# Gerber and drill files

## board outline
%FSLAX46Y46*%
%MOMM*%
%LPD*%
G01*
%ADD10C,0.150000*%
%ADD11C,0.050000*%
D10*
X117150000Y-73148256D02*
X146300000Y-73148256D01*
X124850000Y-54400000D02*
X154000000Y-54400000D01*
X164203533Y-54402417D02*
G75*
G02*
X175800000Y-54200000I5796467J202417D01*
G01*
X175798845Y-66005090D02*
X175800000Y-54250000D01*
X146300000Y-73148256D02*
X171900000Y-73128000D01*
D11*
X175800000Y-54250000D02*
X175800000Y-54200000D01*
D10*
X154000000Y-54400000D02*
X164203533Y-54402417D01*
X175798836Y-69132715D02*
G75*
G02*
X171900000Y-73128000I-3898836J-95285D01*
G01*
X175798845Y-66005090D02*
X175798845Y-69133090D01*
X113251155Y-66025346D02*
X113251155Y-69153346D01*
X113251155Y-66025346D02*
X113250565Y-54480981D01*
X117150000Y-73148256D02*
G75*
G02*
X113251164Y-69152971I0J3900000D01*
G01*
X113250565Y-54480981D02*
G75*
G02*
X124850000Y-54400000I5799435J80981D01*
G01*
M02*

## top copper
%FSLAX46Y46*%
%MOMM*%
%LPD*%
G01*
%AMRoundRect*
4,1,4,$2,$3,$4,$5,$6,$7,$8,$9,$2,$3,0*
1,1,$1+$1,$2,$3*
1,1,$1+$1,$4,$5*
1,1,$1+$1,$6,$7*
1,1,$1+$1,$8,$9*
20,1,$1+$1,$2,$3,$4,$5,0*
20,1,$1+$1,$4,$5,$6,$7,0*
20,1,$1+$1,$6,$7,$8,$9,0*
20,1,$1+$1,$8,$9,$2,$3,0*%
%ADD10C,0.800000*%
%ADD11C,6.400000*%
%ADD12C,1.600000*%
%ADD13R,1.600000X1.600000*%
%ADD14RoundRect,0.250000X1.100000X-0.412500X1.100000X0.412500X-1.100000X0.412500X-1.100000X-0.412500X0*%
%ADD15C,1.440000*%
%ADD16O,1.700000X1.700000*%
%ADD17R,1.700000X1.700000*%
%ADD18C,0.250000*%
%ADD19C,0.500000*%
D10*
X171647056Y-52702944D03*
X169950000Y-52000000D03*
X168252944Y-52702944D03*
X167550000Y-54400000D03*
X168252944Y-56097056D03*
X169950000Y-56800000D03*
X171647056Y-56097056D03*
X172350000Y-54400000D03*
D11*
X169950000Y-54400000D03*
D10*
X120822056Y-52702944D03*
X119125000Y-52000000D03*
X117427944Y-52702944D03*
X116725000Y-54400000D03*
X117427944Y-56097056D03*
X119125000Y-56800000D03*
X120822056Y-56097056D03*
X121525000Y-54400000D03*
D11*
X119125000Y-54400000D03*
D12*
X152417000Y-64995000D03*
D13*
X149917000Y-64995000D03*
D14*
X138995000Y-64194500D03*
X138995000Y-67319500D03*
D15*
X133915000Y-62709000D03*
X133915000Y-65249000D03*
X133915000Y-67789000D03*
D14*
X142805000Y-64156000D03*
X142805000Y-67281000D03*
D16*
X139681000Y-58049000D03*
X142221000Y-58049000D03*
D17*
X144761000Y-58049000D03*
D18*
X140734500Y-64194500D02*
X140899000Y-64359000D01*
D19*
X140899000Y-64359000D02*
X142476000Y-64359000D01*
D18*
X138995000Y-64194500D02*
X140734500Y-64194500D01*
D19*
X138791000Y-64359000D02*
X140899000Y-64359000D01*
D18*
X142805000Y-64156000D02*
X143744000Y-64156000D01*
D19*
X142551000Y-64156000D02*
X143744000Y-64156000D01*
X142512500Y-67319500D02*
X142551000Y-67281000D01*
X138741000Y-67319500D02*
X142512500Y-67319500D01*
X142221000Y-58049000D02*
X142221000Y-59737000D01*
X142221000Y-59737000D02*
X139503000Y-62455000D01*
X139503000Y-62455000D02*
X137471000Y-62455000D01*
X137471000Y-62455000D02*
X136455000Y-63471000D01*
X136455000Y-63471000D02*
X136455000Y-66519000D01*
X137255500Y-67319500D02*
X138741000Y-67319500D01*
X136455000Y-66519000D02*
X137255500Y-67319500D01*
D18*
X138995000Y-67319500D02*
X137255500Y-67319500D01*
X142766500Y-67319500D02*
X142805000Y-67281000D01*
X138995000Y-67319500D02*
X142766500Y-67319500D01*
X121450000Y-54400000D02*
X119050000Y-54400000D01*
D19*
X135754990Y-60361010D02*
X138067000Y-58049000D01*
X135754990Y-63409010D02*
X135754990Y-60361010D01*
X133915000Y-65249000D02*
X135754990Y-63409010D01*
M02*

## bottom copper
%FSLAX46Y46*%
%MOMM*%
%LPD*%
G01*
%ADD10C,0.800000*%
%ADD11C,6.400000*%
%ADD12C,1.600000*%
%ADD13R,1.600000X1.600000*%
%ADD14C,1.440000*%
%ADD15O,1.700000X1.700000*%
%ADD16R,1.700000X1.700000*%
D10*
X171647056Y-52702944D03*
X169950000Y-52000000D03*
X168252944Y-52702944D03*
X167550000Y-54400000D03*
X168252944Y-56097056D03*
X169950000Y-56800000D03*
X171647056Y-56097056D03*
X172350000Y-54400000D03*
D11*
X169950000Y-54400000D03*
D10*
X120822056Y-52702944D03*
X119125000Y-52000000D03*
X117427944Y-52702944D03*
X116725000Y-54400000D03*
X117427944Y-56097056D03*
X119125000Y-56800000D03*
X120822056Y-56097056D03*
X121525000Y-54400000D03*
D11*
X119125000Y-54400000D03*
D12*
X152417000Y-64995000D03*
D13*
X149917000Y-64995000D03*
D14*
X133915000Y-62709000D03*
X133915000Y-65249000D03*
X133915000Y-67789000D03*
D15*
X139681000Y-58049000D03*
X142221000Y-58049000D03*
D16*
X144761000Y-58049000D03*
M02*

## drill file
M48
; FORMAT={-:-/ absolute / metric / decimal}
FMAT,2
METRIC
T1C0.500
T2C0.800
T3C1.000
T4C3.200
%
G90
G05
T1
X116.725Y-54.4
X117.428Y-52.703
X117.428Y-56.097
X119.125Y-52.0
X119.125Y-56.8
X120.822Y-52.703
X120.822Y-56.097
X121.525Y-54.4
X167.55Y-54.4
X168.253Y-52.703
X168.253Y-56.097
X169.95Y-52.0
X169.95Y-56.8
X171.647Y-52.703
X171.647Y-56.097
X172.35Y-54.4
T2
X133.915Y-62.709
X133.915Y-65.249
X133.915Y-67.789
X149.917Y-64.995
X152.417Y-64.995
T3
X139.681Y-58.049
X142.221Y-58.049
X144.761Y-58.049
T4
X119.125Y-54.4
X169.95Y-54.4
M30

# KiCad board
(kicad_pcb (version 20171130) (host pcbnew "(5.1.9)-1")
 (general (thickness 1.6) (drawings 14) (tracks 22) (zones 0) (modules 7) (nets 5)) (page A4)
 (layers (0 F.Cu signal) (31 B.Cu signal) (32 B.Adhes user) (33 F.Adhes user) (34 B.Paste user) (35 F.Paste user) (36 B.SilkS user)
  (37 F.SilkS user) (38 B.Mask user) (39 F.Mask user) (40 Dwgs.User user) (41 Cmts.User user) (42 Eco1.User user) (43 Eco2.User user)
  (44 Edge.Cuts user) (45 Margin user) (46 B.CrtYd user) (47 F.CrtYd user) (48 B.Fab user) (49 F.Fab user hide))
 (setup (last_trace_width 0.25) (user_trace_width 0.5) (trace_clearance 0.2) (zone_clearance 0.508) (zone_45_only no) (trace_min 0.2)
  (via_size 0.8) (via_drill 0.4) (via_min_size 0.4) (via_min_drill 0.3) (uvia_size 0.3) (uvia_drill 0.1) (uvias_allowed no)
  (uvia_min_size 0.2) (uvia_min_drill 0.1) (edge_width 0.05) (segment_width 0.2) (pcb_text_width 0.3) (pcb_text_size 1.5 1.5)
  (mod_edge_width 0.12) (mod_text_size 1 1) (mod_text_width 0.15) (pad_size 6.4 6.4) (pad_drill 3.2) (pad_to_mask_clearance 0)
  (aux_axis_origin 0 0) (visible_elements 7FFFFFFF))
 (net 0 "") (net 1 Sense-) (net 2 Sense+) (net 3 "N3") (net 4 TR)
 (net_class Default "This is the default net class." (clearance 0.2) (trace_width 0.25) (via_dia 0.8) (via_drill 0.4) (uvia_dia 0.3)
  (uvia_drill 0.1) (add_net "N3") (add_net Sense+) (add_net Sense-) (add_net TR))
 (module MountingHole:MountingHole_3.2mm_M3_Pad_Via (layer F.Cu) (at 169.95 54.4)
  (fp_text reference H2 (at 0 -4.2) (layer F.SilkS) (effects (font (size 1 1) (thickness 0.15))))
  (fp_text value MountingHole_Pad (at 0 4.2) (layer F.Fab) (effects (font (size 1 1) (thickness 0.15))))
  (pad 1 thru_hole circle (at 1.697056 -1.697056) (size 0.8 0.8) (drill 0.5) (layers *.Cu *.Mask) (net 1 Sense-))
  (pad 1 thru_hole circle (at 0 -2.4) (size 0.8 0.8) (drill 0.5) (layers *.Cu *.Mask) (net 1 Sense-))
  (pad 1 thru_hole circle (at -1.697056 -1.697056) (size 0.8 0.8) (drill 0.5) (layers *.Cu *.Mask) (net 1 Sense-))
  (pad 1 thru_hole circle (at -2.4 0) (size 0.8 0.8) (drill 0.5) (layers *.Cu *.Mask) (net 1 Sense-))
  (pad 1 thru_hole circle (at -1.697056 1.697056) (size 0.8 0.8) (drill 0.5) (layers *.Cu *.Mask) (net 1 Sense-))
  (pad 1 thru_hole circle (at 0 2.4) (size 0.8 0.8) (drill 0.5) (layers *.Cu *.Mask) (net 1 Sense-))
  (pad 1 thru_hole circle (at 1.697056 1.697056) (size 0.8 0.8) (drill 0.5) (layers *.Cu *.Mask) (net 1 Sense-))
  (pad 1 thru_hole circle (at 2.4 0) (size 0.8 0.8) (drill 0.5) (layers *.Cu *.Mask) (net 1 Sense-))
  (pad 1 thru_hole circle (at 0 0) (size 6.4 6.4) (drill 3.2) (layers *.Cu *.Mask) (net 1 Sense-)))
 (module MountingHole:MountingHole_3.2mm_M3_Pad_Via (layer F.Cu) (at 119.125 54.4)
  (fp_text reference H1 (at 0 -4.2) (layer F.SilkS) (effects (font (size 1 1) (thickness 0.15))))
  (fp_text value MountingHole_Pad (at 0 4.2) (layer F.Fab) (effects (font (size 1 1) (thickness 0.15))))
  (pad 1 thru_hole circle (at 1.697056 -1.697056) (size 0.8 0.8) (drill 0.5) (layers *.Cu *.Mask) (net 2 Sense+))
  (pad 1 thru_hole circle (at 0 -2.4) (size 0.8 0.8) (drill 0.5) (layers *.Cu *.Mask) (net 2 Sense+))
  (pad 1 thru_hole circle (at -1.697056 -1.697056) (size 0.8 0.8) (drill 0.5) (layers *.Cu *.Mask) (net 2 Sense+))
  (pad 1 thru_hole circle (at -2.4 0) (size 0.8 0.8) (drill 0.5) (layers *.Cu *.Mask) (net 2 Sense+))
  (pad 1 thru_hole circle (at -1.697056 1.697056) (size 0.8 0.8) (drill 0.5) (layers *.Cu *.Mask) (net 2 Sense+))
  (pad 1 thru_hole circle (at 0 2.4) (size 0.8 0.8) (drill 0.5) (layers *.Cu *.Mask) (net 2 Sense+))
  (pad 1 thru_hole circle (at 1.697056 1.697056) (size 0.8 0.8) (drill 0.5) (layers *.Cu *.Mask) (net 2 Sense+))
  (pad 1 thru_hole circle (at 2.4 0) (size 0.8 0.8) (drill 0.5) (layers *.Cu *.Mask) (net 2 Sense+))
  (pad 1 thru_hole circle (at 0 0) (size 6.4 6.4) (drill 3.2) (layers *.Cu *.Mask) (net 2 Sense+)))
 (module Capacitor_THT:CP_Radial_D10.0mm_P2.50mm (layer F.Cu) (at 149.917 64.995)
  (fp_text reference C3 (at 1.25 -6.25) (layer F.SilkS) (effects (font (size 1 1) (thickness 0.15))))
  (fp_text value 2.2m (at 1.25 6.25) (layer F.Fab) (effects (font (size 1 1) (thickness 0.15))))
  (pad 2 thru_hole circle (at 2.5 0) (size 1.6 1.6) (drill 0.8) (layers *.Cu *.Mask) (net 1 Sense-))
  (pad 1 thru_hole rect (at 0 0) (size 1.6 1.6) (drill 0.8) (layers *.Cu *.Mask) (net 2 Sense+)))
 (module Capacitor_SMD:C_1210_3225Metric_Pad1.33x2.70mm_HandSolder (layer F.Cu) (at 138.995 65.757 90)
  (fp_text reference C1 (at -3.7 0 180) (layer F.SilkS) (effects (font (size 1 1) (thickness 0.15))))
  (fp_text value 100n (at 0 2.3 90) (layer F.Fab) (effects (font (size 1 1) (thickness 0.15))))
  (pad 2 smd roundrect (at 1.5625 0 90) (size 1.325 2.7) (layers F.Cu F.Paste F.Mask) (roundrect_rratio 0.188679) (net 1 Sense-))
  (pad 1 smd roundrect (at -1.5625 0 90) (size 1.325 2.7) (layers F.Cu F.Paste F.Mask) (roundrect_rratio 0.188679) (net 2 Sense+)))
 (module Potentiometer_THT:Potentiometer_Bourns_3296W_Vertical (layer F.Cu) (at 133.915 67.789 270)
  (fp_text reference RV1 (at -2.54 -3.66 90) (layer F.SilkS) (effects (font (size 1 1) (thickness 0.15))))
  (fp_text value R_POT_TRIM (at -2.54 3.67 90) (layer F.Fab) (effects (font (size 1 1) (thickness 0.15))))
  (pad 3 thru_hole circle (at -5.08 0 270) (size 1.44 1.44) (drill 0.8) (layers *.Cu *.Mask) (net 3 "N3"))
  (pad 2 thru_hole circle (at -2.54 0 270) (size 1.44 1.44) (drill 0.8) (layers *.Cu *.Mask) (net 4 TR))
  (pad 1 thru_hole circle (at 0 0 270) (size 1.44 1.44) (drill 0.8) (layers *.Cu *.Mask) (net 1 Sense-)))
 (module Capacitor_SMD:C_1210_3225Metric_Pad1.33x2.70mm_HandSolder (layer F.Cu) (at 142.805 65.7185 90)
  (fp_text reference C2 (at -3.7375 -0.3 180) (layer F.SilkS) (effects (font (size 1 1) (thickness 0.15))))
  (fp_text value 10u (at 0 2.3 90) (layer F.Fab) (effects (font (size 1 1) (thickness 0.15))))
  (pad 2 smd roundrect (at 1.5625 0 90) (size 1.325 2.7) (layers F.Cu F.Paste F.Mask) (roundrect_rratio 0.188679) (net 1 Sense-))
  (pad 1 smd roundrect (at -1.5625 0 90) (size 1.325 2.7) (layers F.Cu F.Paste F.Mask) (roundrect_rratio 0.188679) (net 2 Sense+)))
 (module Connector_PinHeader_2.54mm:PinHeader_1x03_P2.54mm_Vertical (layer F.Cu) (at 144.761 58.049 270)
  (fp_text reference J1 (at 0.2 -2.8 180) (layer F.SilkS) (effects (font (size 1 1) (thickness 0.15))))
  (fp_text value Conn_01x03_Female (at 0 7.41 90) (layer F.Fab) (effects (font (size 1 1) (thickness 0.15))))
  (pad 3 thru_hole oval (at 0 5.08 270) (size 1.7 1.7) (drill 1) (layers *.Cu *.Mask) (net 4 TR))
  (pad 2 thru_hole oval (at 0 2.54 270) (size 1.7 1.7) (drill 1) (layers *.Cu *.Mask) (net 2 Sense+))
  (pad 1 thru_hole rect (at 0 0 270) (size 1.7 1.7) (drill 1) (layers *.Cu *.Mask) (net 1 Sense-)))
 (gr_line (start 117.15 73.148256) (end 146.3 73.148256) (layer Edge.Cuts) (width 0.15))
 (gr_line (start 124.85 54.4) (end 154 54.4) (layer Edge.Cuts) (width 0.15))
 (gr_arc (start 170 54.2) (end 175.8 54.2) (angle -182) (layer Edge.Cuts) (width 0.15))
 (gr_line (start 175.798845 66.00509) (end 175.8 54.25) (layer Edge.Cuts) (width 0.15))
 (gr_line (start 146.3 73.148256) (end 171.9 73.128) (layer Edge.Cuts) (width 0.15))
 (gr_line (start 175.8 54.25) (end 175.8 54.2) (layer Edge.Cuts) (width 0.05))
 (gr_line (start 154 54.4) (end 164.203533 54.402417) (layer Edge.Cuts) (width 0.15))
 (gr_arc (start 171.9 69.228) (end 171.9 73.128) (angle -91.4) (layer Edge.Cuts) (width 0.15))
 (gr_line (start 175.798845 66.00509) (end 175.798845 69.13309) (layer Edge.Cuts) (width 0.15))
 (gr_line (start 113.251155 66.025346) (end 113.251155 69.153346) (layer Edge.Cuts) (width 0.15))
 (gr_line (start 113.251155 66.025346) (end 113.250565 54.480981) (layer Edge.Cuts) (width 0.15))
 (gr_arc (start 117.15 69.248256) (end 117.15 73.148256) (angle 91.4) (layer Edge.Cuts) (width 0.15))
 (gr_arc (start 119.05 54.4) (end 124.85 54.4) (angle -180.8) (layer Edge.Cuts) (width 0.15))
 (segment (start 140.7345 64.1945) (end 140.899 64.359) (width 0.25) (layer F.Cu) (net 1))
 (segment (start 140.899 64.359) (end 142.476 64.359) (width 0.5) (layer F.Cu) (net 1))
 (segment (start 138.995 64.1945) (end 140.7345 64.1945) (width 0.25) (layer F.Cu) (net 1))
 (segment (start 138.791 64.359) (end 140.899 64.359) (width 0.5) (layer F.Cu) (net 1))
 (segment (start 142.805 64.156) (end 143.744 64.156) (width 0.25) (layer F.Cu) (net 1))
 (segment (start 142.551 64.156) (end 143.744 64.156) (width 0.5) (layer F.Cu) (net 1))
 (segment (start 142.5125 67.3195) (end 142.551 67.281) (width 0.5) (layer F.Cu) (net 2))
 (segment (start 138.741 67.3195) (end 142.5125 67.3195) (width 0.5) (layer F.Cu) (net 2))
 (segment (start 142.221 58.049) (end 142.221 59.737) (width 0.5) (layer F.Cu) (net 2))
 (segment (start 142.221 59.737) (end 139.503 62.455) (width 0.5) (layer F.Cu) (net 2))
 (segment (start 139.503 62.455) (end 137.471 62.455) (width 0.5) (layer F.Cu) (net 2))
 (segment (start 137.471 62.455) (end 136.455 63.471) (width 0.5) (layer F.Cu) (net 2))
 (segment (start 136.455 63.471) (end 136.455 66.519) (width 0.5) (layer F.Cu) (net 2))
 (segment (start 137.2555 67.3195) (end 138.741 67.3195) (width 0.5) (layer F.Cu) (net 2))
 (segment (start 136.455 66.519) (end 137.2555 67.3195) (width 0.5) (layer F.Cu) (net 2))
 (segment (start 138.995 67.3195) (end 137.2555 67.3195) (width 0.25) (layer F.Cu) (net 2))
 (segment (start 142.7665 67.3195) (end 142.805 67.281) (width 0.25) (layer F.Cu) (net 2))
 (segment (start 138.995 67.3195) (end 142.7665 67.3195) (width 0.25) (layer F.Cu) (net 2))
 (segment (start 121.45 54.4) (end 119.05 54.4) (width 0.25) (layer F.Cu) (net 2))
 (segment (start 135.75499 60.36101) (end 138.067 58.049) (width 0.5) (layer F.Cu) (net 4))
 (segment (start 135.75499 63.40901) (end 135.75499 60.36101) (width 0.5) (layer F.Cu) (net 4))
 (segment (start 133.915 65.249) (end 135.75499 63.40901) (width 0.5) (layer F.Cu) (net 4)))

